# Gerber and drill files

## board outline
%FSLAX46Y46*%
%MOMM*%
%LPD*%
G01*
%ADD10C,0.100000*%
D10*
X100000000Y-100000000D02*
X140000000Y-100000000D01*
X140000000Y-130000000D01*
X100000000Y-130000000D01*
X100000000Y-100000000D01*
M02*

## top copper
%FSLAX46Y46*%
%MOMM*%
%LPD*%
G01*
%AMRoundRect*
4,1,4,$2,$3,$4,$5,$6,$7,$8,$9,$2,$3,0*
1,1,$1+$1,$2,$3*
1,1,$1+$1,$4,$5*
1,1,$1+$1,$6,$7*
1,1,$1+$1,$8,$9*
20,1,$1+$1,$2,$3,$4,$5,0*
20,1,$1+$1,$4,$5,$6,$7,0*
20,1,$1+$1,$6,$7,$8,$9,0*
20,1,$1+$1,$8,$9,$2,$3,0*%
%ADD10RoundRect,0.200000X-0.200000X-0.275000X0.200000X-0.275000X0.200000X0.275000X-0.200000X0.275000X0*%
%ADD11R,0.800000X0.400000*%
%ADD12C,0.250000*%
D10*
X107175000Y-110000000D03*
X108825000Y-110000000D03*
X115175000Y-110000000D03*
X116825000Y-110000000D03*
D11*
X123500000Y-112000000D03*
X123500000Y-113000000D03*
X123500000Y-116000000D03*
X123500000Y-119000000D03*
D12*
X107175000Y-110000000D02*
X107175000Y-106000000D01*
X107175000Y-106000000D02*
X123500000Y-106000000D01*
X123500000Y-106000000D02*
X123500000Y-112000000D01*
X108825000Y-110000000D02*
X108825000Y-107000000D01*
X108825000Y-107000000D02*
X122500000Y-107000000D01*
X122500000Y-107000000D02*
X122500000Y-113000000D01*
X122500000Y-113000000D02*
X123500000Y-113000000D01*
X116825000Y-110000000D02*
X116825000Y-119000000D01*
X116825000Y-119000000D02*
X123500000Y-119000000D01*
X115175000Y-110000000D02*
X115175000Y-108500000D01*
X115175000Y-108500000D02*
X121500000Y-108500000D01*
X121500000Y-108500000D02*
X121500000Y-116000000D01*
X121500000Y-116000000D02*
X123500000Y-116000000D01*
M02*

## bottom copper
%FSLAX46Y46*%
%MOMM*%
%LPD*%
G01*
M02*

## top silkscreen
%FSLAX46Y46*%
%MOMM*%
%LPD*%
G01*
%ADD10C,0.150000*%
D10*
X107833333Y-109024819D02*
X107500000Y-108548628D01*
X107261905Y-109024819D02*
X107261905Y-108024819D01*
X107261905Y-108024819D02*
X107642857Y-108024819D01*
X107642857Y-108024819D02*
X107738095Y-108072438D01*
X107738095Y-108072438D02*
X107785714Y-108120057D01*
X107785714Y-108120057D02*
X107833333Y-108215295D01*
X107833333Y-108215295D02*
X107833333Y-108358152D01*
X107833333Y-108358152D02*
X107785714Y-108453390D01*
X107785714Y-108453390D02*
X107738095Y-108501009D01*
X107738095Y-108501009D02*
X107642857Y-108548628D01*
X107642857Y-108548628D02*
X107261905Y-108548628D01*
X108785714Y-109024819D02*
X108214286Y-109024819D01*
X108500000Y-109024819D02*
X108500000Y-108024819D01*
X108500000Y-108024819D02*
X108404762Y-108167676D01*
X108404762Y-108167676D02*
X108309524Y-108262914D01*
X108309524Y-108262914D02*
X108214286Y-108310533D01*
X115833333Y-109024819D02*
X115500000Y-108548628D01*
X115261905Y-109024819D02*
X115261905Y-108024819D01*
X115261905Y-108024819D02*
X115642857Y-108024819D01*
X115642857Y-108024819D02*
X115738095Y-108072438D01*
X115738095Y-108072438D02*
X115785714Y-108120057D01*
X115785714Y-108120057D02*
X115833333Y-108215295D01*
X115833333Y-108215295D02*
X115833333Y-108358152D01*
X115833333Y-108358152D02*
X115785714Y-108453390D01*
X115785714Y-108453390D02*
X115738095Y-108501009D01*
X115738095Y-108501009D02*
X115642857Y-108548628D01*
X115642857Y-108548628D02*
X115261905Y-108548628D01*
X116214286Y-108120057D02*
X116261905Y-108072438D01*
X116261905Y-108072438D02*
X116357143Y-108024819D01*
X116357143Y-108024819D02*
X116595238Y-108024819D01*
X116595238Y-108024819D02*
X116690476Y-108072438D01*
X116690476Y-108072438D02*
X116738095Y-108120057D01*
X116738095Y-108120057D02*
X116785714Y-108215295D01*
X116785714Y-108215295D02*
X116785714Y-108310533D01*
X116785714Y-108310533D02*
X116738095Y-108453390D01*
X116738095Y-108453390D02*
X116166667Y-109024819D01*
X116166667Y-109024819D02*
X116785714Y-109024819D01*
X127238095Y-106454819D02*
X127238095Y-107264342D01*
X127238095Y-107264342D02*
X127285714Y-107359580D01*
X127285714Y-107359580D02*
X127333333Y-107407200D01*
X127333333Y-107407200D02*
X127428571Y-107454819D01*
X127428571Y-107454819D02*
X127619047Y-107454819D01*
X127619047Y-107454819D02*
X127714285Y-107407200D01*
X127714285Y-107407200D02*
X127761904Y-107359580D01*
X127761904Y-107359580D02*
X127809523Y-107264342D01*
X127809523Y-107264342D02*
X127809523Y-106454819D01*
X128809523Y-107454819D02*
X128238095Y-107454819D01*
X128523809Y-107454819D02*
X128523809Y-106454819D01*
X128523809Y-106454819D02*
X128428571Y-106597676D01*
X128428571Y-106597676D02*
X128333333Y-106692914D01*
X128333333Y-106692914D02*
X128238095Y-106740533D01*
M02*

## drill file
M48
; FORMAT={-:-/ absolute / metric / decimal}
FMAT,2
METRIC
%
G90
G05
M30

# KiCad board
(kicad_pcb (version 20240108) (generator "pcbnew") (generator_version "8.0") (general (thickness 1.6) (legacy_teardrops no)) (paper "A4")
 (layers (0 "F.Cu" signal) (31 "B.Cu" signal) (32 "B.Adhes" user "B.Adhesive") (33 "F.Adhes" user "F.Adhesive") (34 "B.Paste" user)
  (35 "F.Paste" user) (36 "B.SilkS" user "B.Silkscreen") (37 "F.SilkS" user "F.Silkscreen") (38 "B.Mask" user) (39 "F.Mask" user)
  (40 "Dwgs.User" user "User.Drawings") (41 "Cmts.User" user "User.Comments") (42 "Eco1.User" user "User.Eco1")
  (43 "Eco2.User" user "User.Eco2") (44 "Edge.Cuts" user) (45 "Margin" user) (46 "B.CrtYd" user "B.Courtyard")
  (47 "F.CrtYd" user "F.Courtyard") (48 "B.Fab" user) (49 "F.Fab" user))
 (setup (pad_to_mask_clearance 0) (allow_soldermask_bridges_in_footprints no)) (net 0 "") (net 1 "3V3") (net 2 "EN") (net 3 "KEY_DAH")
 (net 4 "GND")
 (gr_rect (start 100 100) (end 140 130) (stroke (width 0.1) (type default)) (layer "Edge.Cuts"))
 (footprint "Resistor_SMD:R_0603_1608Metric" (layer "F.Cu") (at 108 110)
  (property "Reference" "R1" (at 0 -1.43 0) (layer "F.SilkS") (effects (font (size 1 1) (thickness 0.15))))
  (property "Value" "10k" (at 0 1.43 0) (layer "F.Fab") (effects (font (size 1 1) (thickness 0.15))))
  (pad "1" smd roundrect (at -0.825 0) (size 0.8 0.95) (layers "F.Cu" "F.Paste" "F.Mask") (roundrect_rratio 0.25) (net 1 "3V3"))
  (pad "2" smd roundrect (at 0.825 0) (size 0.8 0.95) (layers "F.Cu" "F.Paste" "F.Mask") (roundrect_rratio 0.25) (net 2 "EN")))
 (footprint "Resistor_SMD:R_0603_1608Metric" (layer "F.Cu") (at 116 110)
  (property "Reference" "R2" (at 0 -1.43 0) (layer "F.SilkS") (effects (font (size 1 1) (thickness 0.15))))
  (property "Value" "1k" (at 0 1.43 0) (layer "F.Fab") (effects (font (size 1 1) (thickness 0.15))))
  (pad "1" smd roundrect (at -0.825 0) (size 0.8 0.95) (layers "F.Cu" "F.Paste" "F.Mask") (roundrect_rratio 0.25) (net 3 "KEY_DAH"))
  (pad "2" smd roundrect (at 0.825 0) (size 0.8 0.95) (layers "F.Cu" "F.Paste" "F.Mask") (roundrect_rratio 0.25) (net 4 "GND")))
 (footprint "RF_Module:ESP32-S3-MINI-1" (layer "F.Cu") (at 128 115)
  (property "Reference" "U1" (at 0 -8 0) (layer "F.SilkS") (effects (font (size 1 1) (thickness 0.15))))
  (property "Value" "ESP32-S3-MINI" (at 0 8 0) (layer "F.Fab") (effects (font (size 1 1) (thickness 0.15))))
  (pad "1" smd rect (at -4.5 -3.0) (size 0.8 0.4) (layers "F.Cu" "F.Paste" "F.Mask") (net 1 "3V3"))
  (pad "2" smd rect (at -4.5 -2.0) (size 0.8 0.4) (layers "F.Cu" "F.Paste" "F.Mask") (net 2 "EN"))
  (pad "5" smd rect (at -4.5 1.0) (size 0.8 0.4) (layers "F.Cu" "F.Paste" "F.Mask") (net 3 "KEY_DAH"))
  (pad "8" smd rect (at -4.5 4.0) (size 0.8 0.4) (layers "F.Cu" "F.Paste" "F.Mask") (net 4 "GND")))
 (segment (start 107.175 110) (end 107.175 106) (width 0.25) (layer "F.Cu") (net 1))
 (segment (start 107.175 106) (end 123.5 106) (width 0.25) (layer "F.Cu") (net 1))
 (segment (start 123.5 106) (end 123.5 112) (width 0.25) (layer "F.Cu") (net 1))
 (segment (start 108.825 110) (end 108.825 107) (width 0.25) (layer "F.Cu") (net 2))
 (segment (start 108.825 107) (end 122.5 107) (width 0.25) (layer "F.Cu") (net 2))
 (segment (start 122.5 107) (end 122.5 113) (width 0.25) (layer "F.Cu") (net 2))
 (segment (start 122.5 113) (end 123.5 113) (width 0.25) (layer "F.Cu") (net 2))
 (segment (start 116.825 110) (end 116.825 119) (width 0.25) (layer "F.Cu") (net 4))
 (segment (start 116.825 119) (end 123.5 119) (width 0.25) (layer "F.Cu") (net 4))
 (segment (start 115.175 110) (end 115.175 108.5) (width 0.25) (layer "F.Cu") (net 3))
 (segment (start 115.175 108.5) (end 121.5 108.5) (width 0.25) (layer "F.Cu") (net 3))
 (segment (start 121.5 108.5) (end 121.5 116) (width 0.25) (layer "F.Cu") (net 3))
 (segment (start 121.5 116) (end 123.5 116) (width 0.25) (layer "F.Cu") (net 3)))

